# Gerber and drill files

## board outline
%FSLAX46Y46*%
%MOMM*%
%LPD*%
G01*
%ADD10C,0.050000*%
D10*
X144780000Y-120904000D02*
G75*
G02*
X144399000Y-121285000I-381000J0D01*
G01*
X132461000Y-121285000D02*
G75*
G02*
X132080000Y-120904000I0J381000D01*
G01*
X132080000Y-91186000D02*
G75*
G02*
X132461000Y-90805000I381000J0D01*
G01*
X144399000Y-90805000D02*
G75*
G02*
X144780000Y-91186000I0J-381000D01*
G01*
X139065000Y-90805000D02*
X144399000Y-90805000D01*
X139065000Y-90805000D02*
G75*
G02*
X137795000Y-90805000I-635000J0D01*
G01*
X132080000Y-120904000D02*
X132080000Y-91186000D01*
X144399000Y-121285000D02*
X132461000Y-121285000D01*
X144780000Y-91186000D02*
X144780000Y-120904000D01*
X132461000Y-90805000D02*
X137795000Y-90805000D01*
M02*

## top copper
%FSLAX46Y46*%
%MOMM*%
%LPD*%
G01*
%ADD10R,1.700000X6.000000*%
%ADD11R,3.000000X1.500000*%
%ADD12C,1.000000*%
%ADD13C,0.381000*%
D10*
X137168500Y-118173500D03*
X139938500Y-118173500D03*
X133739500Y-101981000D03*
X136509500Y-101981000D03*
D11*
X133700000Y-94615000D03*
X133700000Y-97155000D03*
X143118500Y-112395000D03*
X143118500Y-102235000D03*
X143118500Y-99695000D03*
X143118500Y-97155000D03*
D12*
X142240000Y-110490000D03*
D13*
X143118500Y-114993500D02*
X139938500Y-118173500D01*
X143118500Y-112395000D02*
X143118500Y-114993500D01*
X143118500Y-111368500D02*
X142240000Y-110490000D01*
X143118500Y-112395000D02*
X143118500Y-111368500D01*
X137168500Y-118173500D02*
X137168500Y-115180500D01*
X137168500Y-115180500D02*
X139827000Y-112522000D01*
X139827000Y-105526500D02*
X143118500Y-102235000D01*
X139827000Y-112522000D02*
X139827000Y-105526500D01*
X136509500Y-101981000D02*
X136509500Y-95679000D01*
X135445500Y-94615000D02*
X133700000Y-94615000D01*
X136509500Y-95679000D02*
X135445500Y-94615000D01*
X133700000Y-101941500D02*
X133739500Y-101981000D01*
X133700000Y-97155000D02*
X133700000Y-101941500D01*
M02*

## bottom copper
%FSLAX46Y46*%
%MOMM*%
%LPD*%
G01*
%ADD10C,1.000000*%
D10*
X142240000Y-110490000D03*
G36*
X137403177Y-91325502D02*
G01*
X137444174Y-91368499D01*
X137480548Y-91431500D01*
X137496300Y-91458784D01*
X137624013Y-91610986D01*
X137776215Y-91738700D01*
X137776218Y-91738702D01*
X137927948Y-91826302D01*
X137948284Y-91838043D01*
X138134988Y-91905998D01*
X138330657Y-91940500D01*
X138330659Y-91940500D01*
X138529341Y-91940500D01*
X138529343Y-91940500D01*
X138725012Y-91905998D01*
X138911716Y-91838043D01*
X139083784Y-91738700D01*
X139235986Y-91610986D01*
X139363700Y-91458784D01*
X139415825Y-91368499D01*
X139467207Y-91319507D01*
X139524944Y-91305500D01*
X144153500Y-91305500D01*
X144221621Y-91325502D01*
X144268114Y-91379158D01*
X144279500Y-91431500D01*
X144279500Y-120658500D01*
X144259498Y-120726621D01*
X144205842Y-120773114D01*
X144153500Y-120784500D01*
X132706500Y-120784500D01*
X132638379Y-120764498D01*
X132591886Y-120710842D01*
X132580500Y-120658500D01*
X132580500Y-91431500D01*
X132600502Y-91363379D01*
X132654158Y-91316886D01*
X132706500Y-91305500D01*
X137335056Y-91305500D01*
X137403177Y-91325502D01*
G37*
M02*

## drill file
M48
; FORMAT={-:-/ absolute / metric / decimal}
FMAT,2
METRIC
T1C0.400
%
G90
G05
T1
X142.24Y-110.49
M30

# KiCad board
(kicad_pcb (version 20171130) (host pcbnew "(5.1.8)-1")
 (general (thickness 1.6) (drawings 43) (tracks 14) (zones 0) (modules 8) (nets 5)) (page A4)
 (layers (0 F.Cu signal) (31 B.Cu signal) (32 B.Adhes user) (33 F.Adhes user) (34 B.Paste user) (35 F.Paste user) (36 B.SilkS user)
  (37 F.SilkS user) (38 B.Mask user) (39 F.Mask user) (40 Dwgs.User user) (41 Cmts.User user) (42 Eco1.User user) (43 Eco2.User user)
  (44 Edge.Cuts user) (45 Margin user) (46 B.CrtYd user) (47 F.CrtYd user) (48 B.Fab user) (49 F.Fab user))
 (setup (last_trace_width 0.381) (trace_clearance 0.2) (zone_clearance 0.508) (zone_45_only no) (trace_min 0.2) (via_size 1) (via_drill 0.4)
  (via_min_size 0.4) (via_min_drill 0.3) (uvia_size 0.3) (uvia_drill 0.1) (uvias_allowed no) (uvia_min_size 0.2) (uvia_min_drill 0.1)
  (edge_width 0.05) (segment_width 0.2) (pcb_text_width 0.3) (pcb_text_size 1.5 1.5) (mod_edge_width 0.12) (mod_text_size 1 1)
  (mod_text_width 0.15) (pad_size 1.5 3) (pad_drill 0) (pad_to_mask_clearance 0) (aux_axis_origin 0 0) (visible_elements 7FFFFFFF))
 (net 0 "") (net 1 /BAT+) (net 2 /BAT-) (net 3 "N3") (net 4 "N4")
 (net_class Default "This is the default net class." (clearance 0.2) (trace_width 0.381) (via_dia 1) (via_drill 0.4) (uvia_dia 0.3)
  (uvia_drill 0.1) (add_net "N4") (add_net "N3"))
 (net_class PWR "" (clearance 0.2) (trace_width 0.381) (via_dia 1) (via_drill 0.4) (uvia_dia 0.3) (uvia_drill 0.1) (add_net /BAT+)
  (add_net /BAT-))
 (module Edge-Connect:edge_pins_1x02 (layer F.Cu) (at 138.557 118.11)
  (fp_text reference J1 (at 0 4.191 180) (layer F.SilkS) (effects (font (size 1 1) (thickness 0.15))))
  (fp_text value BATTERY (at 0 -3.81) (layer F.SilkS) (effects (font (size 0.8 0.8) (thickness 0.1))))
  (pad 2 smd rect (at -1.3885 0.0635 180) (size 1.7 6) (layers F.Cu F.Paste F.Mask) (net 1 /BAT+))
  (pad 1 smd rect (at 1.3815 0.0635 180) (size 1.7 6) (layers F.Cu F.Paste F.Mask) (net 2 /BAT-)))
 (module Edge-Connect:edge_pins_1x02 (layer F.Cu) (at 135.128 101.9175)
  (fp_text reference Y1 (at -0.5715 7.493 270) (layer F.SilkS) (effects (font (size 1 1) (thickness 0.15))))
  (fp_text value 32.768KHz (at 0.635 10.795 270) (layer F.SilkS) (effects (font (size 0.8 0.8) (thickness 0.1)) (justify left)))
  (pad 2 smd rect (at -1.3885 0.0635 180) (size 1.7 6) (layers F.Cu F.Paste F.Mask) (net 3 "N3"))
  (pad 1 smd rect (at 1.3815 0.0635 180) (size 1.7 6) (layers F.Cu F.Paste F.Mask) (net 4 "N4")))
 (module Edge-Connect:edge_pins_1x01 (layer F.Cu) (at 133.4135 94.615 270)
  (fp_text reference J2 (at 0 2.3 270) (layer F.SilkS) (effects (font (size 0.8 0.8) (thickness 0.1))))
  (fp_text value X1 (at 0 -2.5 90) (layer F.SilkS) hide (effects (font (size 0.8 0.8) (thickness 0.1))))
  (pad 1 smd rect (at 0 -0.2865 90) (size 1.5 3) (layers F.Cu F.Paste F.Mask) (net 4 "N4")))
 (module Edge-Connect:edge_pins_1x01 (layer F.Cu) (at 133.4135 97.155 270)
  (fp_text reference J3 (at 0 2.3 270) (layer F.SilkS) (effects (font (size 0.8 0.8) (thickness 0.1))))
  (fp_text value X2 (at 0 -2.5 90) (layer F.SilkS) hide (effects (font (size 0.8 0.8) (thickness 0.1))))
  (pad 1 smd rect (at 0 -0.2865 90) (size 1.5 3) (layers F.Cu F.Paste F.Mask) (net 3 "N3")))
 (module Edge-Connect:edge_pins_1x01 (layer F.Cu) (at 143.405 112.395 90)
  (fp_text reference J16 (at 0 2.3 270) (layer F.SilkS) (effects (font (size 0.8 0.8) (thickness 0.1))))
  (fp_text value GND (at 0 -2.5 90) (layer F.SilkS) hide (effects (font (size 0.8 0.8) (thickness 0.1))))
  (pad 1 smd rect (at 0 -0.2865 270) (size 1.5 3) (layers F.Cu F.Paste F.Mask) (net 2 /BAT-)))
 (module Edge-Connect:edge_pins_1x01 (layer F.Cu) (at 143.405 102.235 90)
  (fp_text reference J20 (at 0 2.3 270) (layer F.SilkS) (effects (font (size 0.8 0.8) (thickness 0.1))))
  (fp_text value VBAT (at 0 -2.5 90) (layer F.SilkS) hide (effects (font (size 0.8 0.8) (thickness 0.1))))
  (pad 1 smd rect (at 0 -0.2865 270) (size 1.5 3) (layers F.Cu F.Paste F.Mask) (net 1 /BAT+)))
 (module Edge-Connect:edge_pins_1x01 (layer F.Cu) (at 143.405 99.695 90)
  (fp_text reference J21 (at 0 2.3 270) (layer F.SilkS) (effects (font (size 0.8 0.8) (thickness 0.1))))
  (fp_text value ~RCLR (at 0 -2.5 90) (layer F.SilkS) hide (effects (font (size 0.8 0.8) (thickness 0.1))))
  (pad 1 smd rect (at 0 -0.2865 270) (size 1.5 3) (layers F.Cu F.Paste F.Mask)))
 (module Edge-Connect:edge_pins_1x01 (layer F.Cu) (at 143.405 97.155 90)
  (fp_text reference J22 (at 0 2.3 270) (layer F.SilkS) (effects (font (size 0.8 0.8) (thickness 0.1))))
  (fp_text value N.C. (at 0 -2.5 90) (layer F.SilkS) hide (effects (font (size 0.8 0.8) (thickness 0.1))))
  (pad 1 smd rect (at 0 -0.2865 270) (size 1.5 3) (layers F.Cu F.Paste F.Mask)))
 (gr_arc (start 144.399 120.904) (end 144.399 121.285) (angle -90) (layer Edge.Cuts) (width 0.05))
 (gr_arc (start 132.461 120.904) (end 132.08 120.904) (angle -90) (layer Edge.Cuts) (width 0.05))
 (gr_arc (start 132.461 91.186) (end 132.461 90.805) (angle -90) (layer Edge.Cuts) (width 0.05))
 (gr_arc (start 144.399 91.186) (end 144.78 91.186) (angle -90) (layer Edge.Cuts) (width 0.05))
 (gr_line (start 139.065 90.805) (end 144.399 90.805) (layer Edge.Cuts) (width 0.05))
 (gr_arc (start 138.43 90.805) (end 137.795 90.805) (angle -180) (layer Edge.Cuts) (width 0.05))
 (gr_line (start 132.08 120.904) (end 132.08 91.186) (layer Edge.Cuts) (width 0.05))
 (gr_line (start 144.399 121.285) (end 132.461 121.285) (layer Edge.Cuts) (width 0.05))
 (gr_line (start 144.78 91.186) (end 144.78 120.904) (layer Edge.Cuts) (width 0.05))
 (gr_line (start 132.461 90.805) (end 137.795 90.805) (layer Edge.Cuts) (width 0.05))
 (segment (start 143.1185 114.9935) (end 139.9385 118.1735) (width 0.381) (layer F.Cu) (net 2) (status 20))
 (segment (start 143.1185 112.395) (end 143.1185 114.9935) (width 0.381) (layer F.Cu) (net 2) (status 10))
 (via (at 142.24 110.49) (size 1) (drill 0.4) (layers F.Cu B.Cu) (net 2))
 (segment (start 143.1185 111.3685) (end 142.24 110.49) (width 0.381) (layer F.Cu) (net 2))
 (segment (start 143.1185 112.395) (end 143.1185 111.3685) (width 0.381) (layer F.Cu) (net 2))
 (segment (start 137.1685 118.1735) (end 137.1685 115.1805) (width 0.381) (layer F.Cu) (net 1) (status 30))
 (segment (start 137.1685 115.1805) (end 139.827 112.522) (width 0.381) (layer F.Cu) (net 1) (status 10))
 (segment (start 139.827 105.5265) (end 143.1185 102.235) (width 0.381) (layer F.Cu) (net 1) (status 20))
 (segment (start 139.827 112.522) (end 139.827 105.5265) (width 0.381) (layer F.Cu) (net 1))
 (segment (start 136.5095 101.981) (end 136.5095 95.679) (width 0.381) (layer F.Cu) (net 4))
 (segment (start 135.4455 94.615) (end 133.7 94.615) (width 0.381) (layer F.Cu) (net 4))
 (segment (start 136.5095 95.679) (end 135.4455 94.615) (width 0.381) (layer F.Cu) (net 4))
 (segment (start 133.7 101.9415) (end 133.7395 101.981) (width 0.381) (layer F.Cu) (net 3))
 (segment (start 133.7 97.155) (end 133.7 101.9415) (width 0.381) (layer F.Cu) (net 3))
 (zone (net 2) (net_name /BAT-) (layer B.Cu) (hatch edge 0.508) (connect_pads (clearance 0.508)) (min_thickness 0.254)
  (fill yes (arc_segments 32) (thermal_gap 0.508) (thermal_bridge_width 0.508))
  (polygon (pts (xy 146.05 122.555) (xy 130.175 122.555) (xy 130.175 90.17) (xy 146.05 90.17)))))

